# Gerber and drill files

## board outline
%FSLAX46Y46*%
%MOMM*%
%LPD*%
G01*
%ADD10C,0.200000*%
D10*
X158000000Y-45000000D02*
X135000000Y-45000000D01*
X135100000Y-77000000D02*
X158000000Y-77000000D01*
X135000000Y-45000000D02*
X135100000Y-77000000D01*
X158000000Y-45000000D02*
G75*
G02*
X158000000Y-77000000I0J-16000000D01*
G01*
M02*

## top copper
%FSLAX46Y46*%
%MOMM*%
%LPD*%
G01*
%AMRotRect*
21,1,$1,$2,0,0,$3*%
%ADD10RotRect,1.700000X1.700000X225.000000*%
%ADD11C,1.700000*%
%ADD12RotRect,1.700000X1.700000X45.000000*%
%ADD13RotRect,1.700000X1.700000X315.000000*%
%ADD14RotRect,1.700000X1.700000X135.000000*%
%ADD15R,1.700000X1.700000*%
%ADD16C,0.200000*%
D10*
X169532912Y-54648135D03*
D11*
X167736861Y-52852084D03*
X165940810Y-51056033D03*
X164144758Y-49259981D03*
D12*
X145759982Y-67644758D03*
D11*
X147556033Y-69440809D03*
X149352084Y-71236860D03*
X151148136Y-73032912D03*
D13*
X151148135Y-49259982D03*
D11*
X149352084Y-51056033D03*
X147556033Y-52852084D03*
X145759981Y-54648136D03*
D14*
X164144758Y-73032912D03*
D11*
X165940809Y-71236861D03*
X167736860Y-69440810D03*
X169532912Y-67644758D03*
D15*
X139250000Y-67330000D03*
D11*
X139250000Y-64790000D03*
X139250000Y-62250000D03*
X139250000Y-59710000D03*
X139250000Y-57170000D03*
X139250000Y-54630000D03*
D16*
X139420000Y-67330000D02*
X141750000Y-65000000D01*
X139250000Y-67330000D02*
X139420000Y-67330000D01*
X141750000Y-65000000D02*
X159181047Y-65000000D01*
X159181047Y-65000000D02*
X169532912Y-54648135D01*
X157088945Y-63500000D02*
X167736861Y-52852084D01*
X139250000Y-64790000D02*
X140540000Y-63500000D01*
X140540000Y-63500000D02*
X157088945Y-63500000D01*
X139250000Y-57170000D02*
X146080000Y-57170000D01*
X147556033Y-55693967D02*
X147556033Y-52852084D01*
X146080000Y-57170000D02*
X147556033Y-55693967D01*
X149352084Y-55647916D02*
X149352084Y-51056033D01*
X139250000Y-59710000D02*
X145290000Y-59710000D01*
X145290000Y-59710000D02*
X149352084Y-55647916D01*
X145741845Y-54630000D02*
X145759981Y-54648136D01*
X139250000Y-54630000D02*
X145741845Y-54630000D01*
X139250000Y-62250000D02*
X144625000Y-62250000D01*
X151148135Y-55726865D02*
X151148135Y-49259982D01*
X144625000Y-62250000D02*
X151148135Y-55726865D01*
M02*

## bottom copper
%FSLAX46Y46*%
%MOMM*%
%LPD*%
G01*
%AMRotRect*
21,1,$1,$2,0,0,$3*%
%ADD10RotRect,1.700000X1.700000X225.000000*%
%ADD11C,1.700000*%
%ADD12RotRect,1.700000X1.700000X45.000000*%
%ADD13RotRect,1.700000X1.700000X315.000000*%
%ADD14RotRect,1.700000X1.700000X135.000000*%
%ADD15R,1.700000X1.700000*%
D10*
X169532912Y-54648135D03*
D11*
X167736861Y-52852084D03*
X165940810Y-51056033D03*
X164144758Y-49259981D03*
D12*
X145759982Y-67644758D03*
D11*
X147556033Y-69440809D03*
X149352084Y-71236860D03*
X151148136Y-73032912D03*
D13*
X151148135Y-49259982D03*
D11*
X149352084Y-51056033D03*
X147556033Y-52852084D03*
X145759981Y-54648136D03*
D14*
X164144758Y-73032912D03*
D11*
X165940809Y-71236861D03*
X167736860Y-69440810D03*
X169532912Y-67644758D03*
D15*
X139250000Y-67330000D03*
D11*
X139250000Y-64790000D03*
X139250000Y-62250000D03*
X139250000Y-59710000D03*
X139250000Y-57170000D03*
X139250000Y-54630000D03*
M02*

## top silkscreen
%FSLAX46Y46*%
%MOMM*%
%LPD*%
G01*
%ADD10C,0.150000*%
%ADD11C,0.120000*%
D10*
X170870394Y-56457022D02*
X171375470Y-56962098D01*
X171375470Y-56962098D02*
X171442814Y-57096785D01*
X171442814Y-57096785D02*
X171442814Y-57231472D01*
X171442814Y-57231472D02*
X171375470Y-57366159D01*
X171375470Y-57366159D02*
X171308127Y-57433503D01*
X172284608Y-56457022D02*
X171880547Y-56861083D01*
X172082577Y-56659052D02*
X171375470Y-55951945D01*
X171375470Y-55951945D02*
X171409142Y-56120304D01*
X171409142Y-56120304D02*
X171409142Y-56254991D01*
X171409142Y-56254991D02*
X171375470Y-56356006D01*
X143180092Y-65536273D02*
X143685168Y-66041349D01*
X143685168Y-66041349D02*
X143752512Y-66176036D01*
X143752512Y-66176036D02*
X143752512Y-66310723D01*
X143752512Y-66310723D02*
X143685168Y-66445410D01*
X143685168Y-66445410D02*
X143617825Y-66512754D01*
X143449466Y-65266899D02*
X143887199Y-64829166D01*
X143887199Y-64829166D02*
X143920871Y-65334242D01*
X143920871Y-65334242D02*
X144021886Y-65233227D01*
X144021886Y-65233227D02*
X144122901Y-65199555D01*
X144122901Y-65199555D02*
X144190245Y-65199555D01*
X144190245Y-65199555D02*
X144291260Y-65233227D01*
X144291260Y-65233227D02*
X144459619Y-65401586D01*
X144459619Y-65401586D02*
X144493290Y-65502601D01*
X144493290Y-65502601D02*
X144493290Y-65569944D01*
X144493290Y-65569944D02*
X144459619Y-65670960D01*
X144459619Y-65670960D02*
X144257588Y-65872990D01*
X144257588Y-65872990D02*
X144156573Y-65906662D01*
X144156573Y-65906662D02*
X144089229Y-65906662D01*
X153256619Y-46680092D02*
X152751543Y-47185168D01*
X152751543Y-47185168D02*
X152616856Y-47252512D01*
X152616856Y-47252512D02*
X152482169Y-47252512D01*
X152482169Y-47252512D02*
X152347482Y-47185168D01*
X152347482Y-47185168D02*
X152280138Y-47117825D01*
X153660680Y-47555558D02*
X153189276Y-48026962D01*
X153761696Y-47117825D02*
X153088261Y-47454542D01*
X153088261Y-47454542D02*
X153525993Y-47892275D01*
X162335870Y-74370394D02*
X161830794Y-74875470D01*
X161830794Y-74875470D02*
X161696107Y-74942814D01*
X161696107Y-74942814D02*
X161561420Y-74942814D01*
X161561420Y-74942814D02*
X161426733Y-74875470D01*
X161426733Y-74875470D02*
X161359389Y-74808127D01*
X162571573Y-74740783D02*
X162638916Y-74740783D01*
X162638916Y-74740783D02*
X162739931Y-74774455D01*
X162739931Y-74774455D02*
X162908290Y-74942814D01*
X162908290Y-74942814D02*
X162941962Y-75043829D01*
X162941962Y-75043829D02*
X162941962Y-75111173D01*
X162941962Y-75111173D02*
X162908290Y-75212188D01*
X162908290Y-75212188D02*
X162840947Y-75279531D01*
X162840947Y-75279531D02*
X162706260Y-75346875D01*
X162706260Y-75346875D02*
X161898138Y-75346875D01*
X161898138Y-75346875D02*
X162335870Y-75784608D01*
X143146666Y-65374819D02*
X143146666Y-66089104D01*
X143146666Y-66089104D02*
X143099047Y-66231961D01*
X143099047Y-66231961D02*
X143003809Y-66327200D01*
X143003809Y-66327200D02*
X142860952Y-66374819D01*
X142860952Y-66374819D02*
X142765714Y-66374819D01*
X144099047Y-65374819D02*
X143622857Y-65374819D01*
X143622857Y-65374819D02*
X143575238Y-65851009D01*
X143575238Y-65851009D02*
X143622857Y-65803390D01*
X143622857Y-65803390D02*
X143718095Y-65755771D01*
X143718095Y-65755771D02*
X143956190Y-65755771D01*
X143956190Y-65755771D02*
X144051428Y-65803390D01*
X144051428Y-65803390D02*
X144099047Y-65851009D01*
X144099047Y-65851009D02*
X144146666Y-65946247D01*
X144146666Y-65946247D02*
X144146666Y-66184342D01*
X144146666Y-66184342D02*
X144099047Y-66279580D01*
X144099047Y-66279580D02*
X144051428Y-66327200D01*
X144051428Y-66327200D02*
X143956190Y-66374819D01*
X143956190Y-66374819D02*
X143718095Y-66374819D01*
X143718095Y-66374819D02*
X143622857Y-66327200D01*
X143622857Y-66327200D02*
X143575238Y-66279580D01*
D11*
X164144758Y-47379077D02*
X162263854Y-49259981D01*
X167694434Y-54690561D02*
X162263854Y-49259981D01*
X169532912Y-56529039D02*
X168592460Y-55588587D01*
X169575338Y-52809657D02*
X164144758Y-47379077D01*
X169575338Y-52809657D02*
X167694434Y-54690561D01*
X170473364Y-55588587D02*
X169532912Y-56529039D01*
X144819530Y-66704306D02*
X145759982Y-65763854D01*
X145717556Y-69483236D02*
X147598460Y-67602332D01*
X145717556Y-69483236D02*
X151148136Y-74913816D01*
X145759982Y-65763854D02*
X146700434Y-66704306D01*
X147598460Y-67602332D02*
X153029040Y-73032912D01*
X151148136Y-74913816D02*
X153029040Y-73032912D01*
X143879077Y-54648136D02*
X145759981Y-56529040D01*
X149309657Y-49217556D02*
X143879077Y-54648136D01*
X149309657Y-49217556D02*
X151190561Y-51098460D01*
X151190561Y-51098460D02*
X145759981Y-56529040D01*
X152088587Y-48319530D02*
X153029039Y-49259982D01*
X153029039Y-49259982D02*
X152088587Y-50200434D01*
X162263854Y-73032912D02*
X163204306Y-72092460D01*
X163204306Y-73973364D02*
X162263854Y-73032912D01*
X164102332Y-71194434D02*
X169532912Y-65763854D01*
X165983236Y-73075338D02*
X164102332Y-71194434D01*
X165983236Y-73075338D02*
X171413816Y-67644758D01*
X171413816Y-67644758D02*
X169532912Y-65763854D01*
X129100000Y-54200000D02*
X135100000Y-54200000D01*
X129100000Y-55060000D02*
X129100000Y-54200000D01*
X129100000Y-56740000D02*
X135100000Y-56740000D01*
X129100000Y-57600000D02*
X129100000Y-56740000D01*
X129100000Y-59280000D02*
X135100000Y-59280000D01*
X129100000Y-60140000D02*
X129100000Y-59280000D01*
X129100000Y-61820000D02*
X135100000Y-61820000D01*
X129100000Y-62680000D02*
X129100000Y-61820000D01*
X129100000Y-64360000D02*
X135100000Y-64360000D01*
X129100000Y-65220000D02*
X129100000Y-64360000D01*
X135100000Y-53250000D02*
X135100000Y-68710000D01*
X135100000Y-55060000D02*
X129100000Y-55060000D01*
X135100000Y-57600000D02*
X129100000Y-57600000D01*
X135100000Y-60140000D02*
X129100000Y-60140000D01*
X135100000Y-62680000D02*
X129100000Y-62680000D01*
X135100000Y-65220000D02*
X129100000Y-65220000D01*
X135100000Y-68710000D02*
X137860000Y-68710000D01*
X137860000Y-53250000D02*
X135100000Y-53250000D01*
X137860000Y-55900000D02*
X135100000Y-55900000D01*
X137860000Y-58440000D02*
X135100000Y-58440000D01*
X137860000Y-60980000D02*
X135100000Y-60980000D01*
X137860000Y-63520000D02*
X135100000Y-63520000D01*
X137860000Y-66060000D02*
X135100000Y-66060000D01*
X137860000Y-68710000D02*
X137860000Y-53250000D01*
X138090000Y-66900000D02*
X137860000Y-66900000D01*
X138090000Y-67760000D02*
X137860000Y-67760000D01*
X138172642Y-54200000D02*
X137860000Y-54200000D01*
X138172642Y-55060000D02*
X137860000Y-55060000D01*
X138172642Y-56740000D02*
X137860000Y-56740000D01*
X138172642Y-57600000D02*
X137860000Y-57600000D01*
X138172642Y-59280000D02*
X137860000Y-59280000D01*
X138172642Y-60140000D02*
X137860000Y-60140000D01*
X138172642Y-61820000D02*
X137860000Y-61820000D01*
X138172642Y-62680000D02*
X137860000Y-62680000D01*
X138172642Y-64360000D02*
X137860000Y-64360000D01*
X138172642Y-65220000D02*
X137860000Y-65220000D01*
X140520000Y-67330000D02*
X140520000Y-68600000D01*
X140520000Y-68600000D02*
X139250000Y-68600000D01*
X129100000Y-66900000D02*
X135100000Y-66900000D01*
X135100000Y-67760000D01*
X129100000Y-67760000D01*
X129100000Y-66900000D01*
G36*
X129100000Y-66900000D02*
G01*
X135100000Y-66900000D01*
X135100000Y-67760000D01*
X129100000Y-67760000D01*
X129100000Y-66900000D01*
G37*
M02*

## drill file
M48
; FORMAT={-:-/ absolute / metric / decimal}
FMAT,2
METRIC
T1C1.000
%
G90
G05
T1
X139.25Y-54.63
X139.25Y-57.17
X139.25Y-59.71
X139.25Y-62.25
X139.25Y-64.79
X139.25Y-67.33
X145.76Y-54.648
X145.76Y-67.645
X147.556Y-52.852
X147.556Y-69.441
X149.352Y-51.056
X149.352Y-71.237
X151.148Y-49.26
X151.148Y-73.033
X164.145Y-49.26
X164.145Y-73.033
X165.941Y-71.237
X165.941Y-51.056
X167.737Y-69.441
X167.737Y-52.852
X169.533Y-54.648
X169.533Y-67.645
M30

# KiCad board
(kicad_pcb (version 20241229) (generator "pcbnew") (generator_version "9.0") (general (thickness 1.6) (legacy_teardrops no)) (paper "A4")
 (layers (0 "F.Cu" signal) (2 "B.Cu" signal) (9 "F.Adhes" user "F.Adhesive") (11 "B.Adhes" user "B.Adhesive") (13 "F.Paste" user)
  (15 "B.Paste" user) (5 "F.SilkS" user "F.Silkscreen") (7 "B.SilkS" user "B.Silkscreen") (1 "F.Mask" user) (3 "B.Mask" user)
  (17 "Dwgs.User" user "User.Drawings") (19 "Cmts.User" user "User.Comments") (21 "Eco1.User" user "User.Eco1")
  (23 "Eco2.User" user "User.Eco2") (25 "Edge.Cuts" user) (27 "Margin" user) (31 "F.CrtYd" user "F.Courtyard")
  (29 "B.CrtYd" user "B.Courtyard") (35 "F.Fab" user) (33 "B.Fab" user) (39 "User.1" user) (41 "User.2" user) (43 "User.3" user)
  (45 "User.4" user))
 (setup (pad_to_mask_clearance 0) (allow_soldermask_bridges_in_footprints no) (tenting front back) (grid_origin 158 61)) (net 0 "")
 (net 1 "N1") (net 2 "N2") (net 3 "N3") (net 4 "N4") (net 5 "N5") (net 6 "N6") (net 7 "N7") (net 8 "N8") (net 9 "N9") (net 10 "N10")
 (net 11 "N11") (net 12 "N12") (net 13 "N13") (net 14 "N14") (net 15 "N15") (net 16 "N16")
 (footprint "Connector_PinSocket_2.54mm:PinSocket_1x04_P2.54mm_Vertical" (layer "F.Cu") (at 169.532912 54.648135 -135)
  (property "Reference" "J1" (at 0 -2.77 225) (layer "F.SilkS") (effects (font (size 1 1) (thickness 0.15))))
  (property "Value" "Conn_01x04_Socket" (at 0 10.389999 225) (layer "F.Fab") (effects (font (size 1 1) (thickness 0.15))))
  (fp_line (start -1.33 8.95) (end 1.33 8.95) (stroke (width 0.12) (type solid)) (layer "F.SilkS"))
  (fp_line (start 1.33 1.270001) (end 1.33 8.95) (stroke (width 0.12) (type solid)) (layer "F.SilkS"))
  (fp_line (start 1.33 -1.33) (end 1.33 0) (stroke (width 0.12) (type solid)) (layer "F.SilkS"))
  (fp_line (start -1.33 1.270001) (end -1.33 8.95) (stroke (width 0.12) (type solid)) (layer "F.SilkS"))
  (fp_line (start -1.33 1.270001) (end 1.33 1.270001) (stroke (width 0.12) (type solid)) (layer "F.SilkS"))
  (fp_line (start 0 -1.33) (end 1.33 -1.33) (stroke (width 0.12) (type solid)) (layer "F.SilkS"))
  (pad "1" thru_hole rect (at 0 0 225) (size 1.7 1.7) (drill 1) (layers "*.Cu" "*.Mask") (remove_unused_layers no) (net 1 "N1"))
  (pad "2" thru_hole circle (at 0 2.54 225) (size 1.7 1.7) (drill 1) (layers "*.Cu" "*.Mask") (remove_unused_layers no) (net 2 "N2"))
  (pad "3" thru_hole circle (at 0 5.079999 225) (size 1.7 1.7) (drill 1) (layers "*.Cu" "*.Mask") (remove_unused_layers no) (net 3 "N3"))
  (pad "4" thru_hole circle (at 0 7.62 225) (size 1.7 1.7) (drill 1) (layers "*.Cu" "*.Mask") (remove_unused_layers no) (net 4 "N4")))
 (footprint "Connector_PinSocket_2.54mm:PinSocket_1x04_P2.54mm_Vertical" (layer "F.Cu") (at 145.759982 67.644758 45)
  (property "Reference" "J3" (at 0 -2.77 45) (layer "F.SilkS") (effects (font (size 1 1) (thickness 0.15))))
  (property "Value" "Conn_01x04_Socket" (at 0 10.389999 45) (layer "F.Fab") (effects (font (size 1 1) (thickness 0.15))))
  (fp_line (start 0 -1.33) (end 1.33 -1.33) (stroke (width 0.12) (type solid)) (layer "F.SilkS"))
  (fp_line (start -1.33 1.270001) (end 1.33 1.270001) (stroke (width 0.12) (type solid)) (layer "F.SilkS"))
  (fp_line (start -1.33 1.270001) (end -1.33 8.95) (stroke (width 0.12) (type solid)) (layer "F.SilkS"))
  (fp_line (start 1.33 -1.33) (end 1.33 0) (stroke (width 0.12) (type solid)) (layer "F.SilkS"))
  (fp_line (start 1.33 1.270001) (end 1.33 8.95) (stroke (width 0.12) (type solid)) (layer "F.SilkS"))
  (fp_line (start -1.33 8.95) (end 1.33 8.95) (stroke (width 0.12) (type solid)) (layer "F.SilkS"))
  (pad "1" thru_hole rect (at 0 0 45) (size 1.7 1.7) (drill 1) (layers "*.Cu" "*.Mask") (remove_unused_layers no) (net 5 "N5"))
  (pad "2" thru_hole circle (at 0 2.54 45) (size 1.7 1.7) (drill 1) (layers "*.Cu" "*.Mask") (remove_unused_layers no) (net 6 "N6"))
  (pad "3" thru_hole circle (at 0 5.079999 45) (size 1.7 1.7) (drill 1) (layers "*.Cu" "*.Mask") (remove_unused_layers no) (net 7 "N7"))
  (pad "4" thru_hole circle (at 0 7.62 45) (size 1.7 1.7) (drill 1) (layers "*.Cu" "*.Mask") (remove_unused_layers no) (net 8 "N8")))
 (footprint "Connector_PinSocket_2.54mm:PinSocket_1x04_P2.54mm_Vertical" (layer "F.Cu") (at 151.148135 49.259982 -45)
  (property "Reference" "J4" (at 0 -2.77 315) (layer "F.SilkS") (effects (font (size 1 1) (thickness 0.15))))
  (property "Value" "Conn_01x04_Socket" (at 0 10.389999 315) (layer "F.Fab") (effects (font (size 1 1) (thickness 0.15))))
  (fp_line (start -1.33 8.95) (end 1.33 8.95) (stroke (width 0.12) (type solid)) (layer "F.SilkS"))
  (fp_line (start -1.33 1.270001) (end -1.33 8.95) (stroke (width 0.12) (type solid)) (layer "F.SilkS"))
  (fp_line (start -1.33 1.270001) (end 1.33 1.270001) (stroke (width 0.12) (type solid)) (layer "F.SilkS"))
  (fp_line (start 1.33 1.270001) (end 1.33 8.95) (stroke (width 0.12) (type solid)) (layer "F.SilkS"))
  (fp_line (start 0 -1.33) (end 1.33 -1.33) (stroke (width 0.12) (type solid)) (layer "F.SilkS"))
  (fp_line (start 1.33 -1.33) (end 1.33 0) (stroke (width 0.12) (type solid)) (layer "F.SilkS"))
  (pad "1" thru_hole rect (at 0 0 315) (size 1.7 1.7) (drill 1) (layers "*.Cu" "*.Mask") (remove_unused_layers no) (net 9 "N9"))
  (pad "2" thru_hole circle (at 0 2.54 315) (size 1.7 1.7) (drill 1) (layers "*.Cu" "*.Mask") (remove_unused_layers no) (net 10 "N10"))
  (pad "3" thru_hole circle (at 0 5.079999 315) (size 1.7 1.7) (drill 1) (layers "*.Cu" "*.Mask") (remove_unused_layers no) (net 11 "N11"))
  (pad "4" thru_hole circle (at 0 7.62 315) (size 1.7 1.7) (drill 1) (layers "*.Cu" "*.Mask") (remove_unused_layers no) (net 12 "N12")))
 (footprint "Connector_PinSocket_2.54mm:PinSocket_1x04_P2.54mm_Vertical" (layer "F.Cu") (at 164.144758 73.032912 135)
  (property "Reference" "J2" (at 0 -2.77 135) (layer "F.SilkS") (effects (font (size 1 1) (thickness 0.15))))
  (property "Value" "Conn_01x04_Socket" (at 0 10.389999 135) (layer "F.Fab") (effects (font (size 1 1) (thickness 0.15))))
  (fp_line (start 1.33 -1.33) (end 1.33 0) (stroke (width 0.12) (type solid)) (layer "F.SilkS"))
  (fp_line (start 0 -1.33) (end 1.33 -1.33) (stroke (width 0.12) (type solid)) (layer "F.SilkS"))
  (fp_line (start 1.33 1.270001) (end 1.33 8.95) (stroke (width 0.12) (type solid)) (layer "F.SilkS"))
  (fp_line (start -1.33 1.270001) (end 1.33 1.270001) (stroke (width 0.12) (type solid)) (layer "F.SilkS"))
  (fp_line (start -1.33 1.270001) (end -1.33 8.95) (stroke (width 0.12) (type solid)) (layer "F.SilkS"))
  (fp_line (start -1.33 8.95) (end 1.33 8.95) (stroke (width 0.12) (type solid)) (layer "F.SilkS"))
  (pad "1" thru_hole rect (at 0 0 135) (size 1.7 1.7) (drill 1) (layers "*.Cu" "*.Mask") (remove_unused_layers no) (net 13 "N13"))
  (pad "2" thru_hole circle (at 0 2.54 135) (size 1.7 1.7) (drill 1) (layers "*.Cu" "*.Mask") (remove_unused_layers no) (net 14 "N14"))
  (pad "3" thru_hole circle (at 0 5.079999 135) (size 1.7 1.7) (drill 1) (layers "*.Cu" "*.Mask") (remove_unused_layers no) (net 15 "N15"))
  (pad "4" thru_hole circle (at 0 7.62 135) (size 1.7 1.7) (drill 1) (layers "*.Cu" "*.Mask") (remove_unused_layers no) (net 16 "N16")))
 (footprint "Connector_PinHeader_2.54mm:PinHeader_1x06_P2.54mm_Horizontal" (layer "F.Cu") (at 139.25 67.33 180)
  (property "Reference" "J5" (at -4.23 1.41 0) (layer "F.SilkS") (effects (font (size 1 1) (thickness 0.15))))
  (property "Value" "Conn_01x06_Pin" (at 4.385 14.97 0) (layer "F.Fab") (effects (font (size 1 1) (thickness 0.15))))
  (fp_line (start 10.15 13.13) (end 4.15 13.13) (stroke (width 0.12) (type solid)) (layer "F.SilkS"))
  (fp_line (start 10.15 12.27) (end 10.15 13.13) (stroke (width 0.12) (type solid)) (layer "F.SilkS"))
  (fp_line (start 10.15 10.59) (end 4.15 10.59) (stroke (width 0.12) (type solid)) (layer "F.SilkS"))
  (fp_line (start 10.15 9.73) (end 10.15 10.59) (stroke (width 0.12) (type solid)) (layer "F.SilkS"))
  (fp_line (start 10.15 8.05) (end 4.15 8.05) (stroke (width 0.12) (type solid)) (layer "F.SilkS"))
  (fp_line (start 10.15 7.19) (end 10.15 8.05) (stroke (width 0.12) (type solid)) (layer "F.SilkS"))
  (fp_line (start 10.15 5.51) (end 4.15 5.51) (stroke (width 0.12) (type solid)) (layer "F.SilkS"))
  (fp_line (start 10.15 4.65) (end 10.15 5.51) (stroke (width 0.12) (type solid)) (layer "F.SilkS"))
  (fp_line (start 10.15 2.97) (end 4.15 2.97) (stroke (width 0.12) (type solid)) (layer "F.SilkS"))
  (fp_line (start 10.15 2.11) (end 10.15 2.97) (stroke (width 0.12) (type solid)) (layer "F.SilkS"))
  (fp_line (start 4.15 14.08) (end 4.15 -1.38) (stroke (width 0.12) (type solid)) (layer "F.SilkS"))
  (fp_line (start 4.15 12.27) (end 10.15 12.27) (stroke (width 0.12) (type solid)) (layer "F.SilkS"))
  (fp_line (start 4.15 9.73) (end 10.15 9.73) (stroke (width 0.12) (type solid)) (layer "F.SilkS"))
  (fp_line (start 4.15 7.19) (end 10.15 7.19) (stroke (width 0.12) (type solid)) (layer "F.SilkS"))
  (fp_line (start 4.15 4.65) (end 10.15 4.65) (stroke (width 0.12) (type solid)) (layer "F.SilkS"))
  (fp_line (start 4.15 2.11) (end 10.15 2.11) (stroke (width 0.12) (type solid)) (layer "F.SilkS"))
  (fp_line (start 4.15 -1.38) (end 1.39 -1.38) (stroke (width 0.12) (type solid)) (layer "F.SilkS"))
  (fp_line (start 1.39 14.08) (end 4.15 14.08) (stroke (width 0.12) (type solid)) (layer "F.SilkS"))
  (fp_line (start 1.39 11.43) (end 4.15 11.43) (stroke (width 0.12) (type solid)) (layer "F.SilkS"))
  (fp_line (start 1.39 8.89) (end 4.15 8.89) (stroke (width 0.12) (type solid)) (layer "F.SilkS"))
  (fp_line (start 1.39 6.35) (end 4.15 6.35) (stroke (width 0.12) (type solid)) (layer "F.SilkS"))
  (fp_line (start 1.39 3.81) (end 4.15 3.81) (stroke (width 0.12) (type solid)) (layer "F.SilkS"))
  (fp_line (start 1.39 1.27) (end 4.15 1.27) (stroke (width 0.12) (type solid)) (layer "F.SilkS"))
  (fp_line (start 1.39 -1.38) (end 1.39 14.08) (stroke (width 0.12) (type solid)) (layer "F.SilkS"))
  (fp_line (start 1.16 0.43) (end 1.39 0.43) (stroke (width 0.12) (type solid)) (layer "F.SilkS"))
  (fp_line (start 1.16 -0.43) (end 1.39 -0.43) (stroke (width 0.12) (type solid)) (layer "F.SilkS"))
  (fp_line (start 1.077358 13.13) (end 1.39 13.13) (stroke (width 0.12) (type solid)) (layer "F.SilkS"))
  (fp_line (start 1.077358 12.27) (end 1.39 12.27) (stroke (width 0.12) (type solid)) (layer "F.SilkS"))
  (fp_line (start 1.077358 10.59) (end 1.39 10.59) (stroke (width 0.12) (type solid)) (layer "F.SilkS"))
  (fp_line (start 1.077358 9.73) (end 1.39 9.73) (stroke (width 0.12) (type solid)) (layer "F.SilkS"))
  (fp_line (start 1.077358 8.05) (end 1.39 8.05) (stroke (width 0.12) (type solid)) (layer "F.SilkS"))
  (fp_line (start 1.077358 7.19) (end 1.39 7.19) (stroke (width 0.12) (type solid)) (layer "F.SilkS"))
  (fp_line (start 1.077358 5.51) (end 1.39 5.51) (stroke (width 0.12) (type solid)) (layer "F.SilkS"))
  (fp_line (start 1.077358 4.65) (end 1.39 4.65) (stroke (width 0.12) (type solid)) (layer "F.SilkS"))
  (fp_line (start 1.077358 2.97) (end 1.39 2.97) (stroke (width 0.12) (type solid)) (layer "F.SilkS"))
  (fp_line (start 1.077358 2.11) (end 1.39 2.11) (stroke (width 0.12) (type solid)) (layer "F.SilkS"))
  (fp_line (start -1.27 0) (end -1.27 -1.27) (stroke (width 0.12) (type solid)) (layer "F.SilkS"))
  (fp_line (start -1.27 -1.27) (end 0 -1.27) (stroke (width 0.12) (type solid)) (layer "F.SilkS"))
  (fp_rect (start 4.15 -0.43) (end 10.15 0.43) (stroke (width 0.12) (type solid)) (fill yes) (layer "F.SilkS"))
  (pad "1" thru_hole rect (at 0 0 180) (size 1.7 1.7) (drill 1) (layers "*.Cu" "*.Mask") (remove_unused_layers no) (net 1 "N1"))
  (pad "2" thru_hole circle (at 0 2.54 180) (size 1.7 1.7) (drill 1) (layers "*.Cu" "*.Mask") (remove_unused_layers no) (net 2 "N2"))
  (pad "3" thru_hole circle (at 0 5.08 180) (size 1.7 1.7) (drill 1) (layers "*.Cu" "*.Mask") (remove_unused_layers no) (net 9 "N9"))
  (pad "4" thru_hole circle (at 0 7.62 180) (size 1.7 1.7) (drill 1) (layers "*.Cu" "*.Mask") (remove_unused_layers no) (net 10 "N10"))
  (pad "5" thru_hole circle (at 0 10.16 180) (size 1.7 1.7) (drill 1) (layers "*.Cu" "*.Mask") (remove_unused_layers no) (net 11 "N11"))
  (pad "6" thru_hole circle (at 0 12.7 180) (size 1.7 1.7) (drill 1) (layers "*.Cu" "*.Mask") (remove_unused_layers no) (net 12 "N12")))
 (gr_line (start 158 45) (end 135 45) (stroke (width 0.2) (type solid)) (layer "Edge.Cuts"))
 (gr_line (start 135.1 77) (end 158 77) (stroke (width 0.2) (type solid)) (layer "Edge.Cuts"))
 (gr_line (start 135 45) (end 135.1 77) (stroke (width 0.2) (type solid)) (layer "Edge.Cuts"))
 (gr_arc (start 158 45) (mid 174 61) (end 158 77) (stroke (width 0.2) (type solid)) (layer "Edge.Cuts"))
 (segment (start 139.42 67.33) (end 141.75 65) (width 0.2) (layer "F.Cu") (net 1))
 (segment (start 139.25 67.33) (end 139.42 67.33) (width 0.2) (layer "F.Cu") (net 1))
 (segment (start 141.75 65) (end 159.181047 65) (width 0.2) (layer "F.Cu") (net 1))
 (segment (start 159.181047 65) (end 169.532912 54.648135) (width 0.2) (layer "F.Cu") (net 1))
 (segment (start 157.088945 63.5) (end 167.736861 52.852084) (width 0.2) (layer "F.Cu") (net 2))
 (segment (start 139.25 64.79) (end 140.54 63.5) (width 0.2) (layer "F.Cu") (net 2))
 (segment (start 140.54 63.5) (end 157.088945 63.5) (width 0.2) (layer "F.Cu") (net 2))
 (segment (start 139.25 57.17) (end 146.08 57.17) (width 0.2) (layer "F.Cu") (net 11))
 (segment (start 147.556033 55.693967) (end 147.556033 52.852084) (width 0.2) (layer "F.Cu") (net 11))
 (segment (start 146.08 57.17) (end 147.556033 55.693967) (width 0.2) (layer "F.Cu") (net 11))
 (segment (start 149.352084 55.647916) (end 149.352084 51.056033) (width 0.2) (layer "F.Cu") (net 10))
 (segment (start 139.25 59.71) (end 145.29 59.71) (width 0.2) (layer "F.Cu") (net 10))
 (segment (start 145.29 59.71) (end 149.352084 55.647916) (width 0.2) (layer "F.Cu") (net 10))
 (segment (start 145.741845 54.63) (end 145.759981 54.648136) (width 0.2) (layer "F.Cu") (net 12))
 (segment (start 139.25 54.63) (end 145.741845 54.63) (width 0.2) (layer "F.Cu") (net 12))
 (segment (start 139.25 62.25) (end 144.625 62.25) (width 0.2) (layer "F.Cu") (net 9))
 (segment (start 151.148135 55.726865) (end 151.148135 49.259982) (width 0.2) (layer "F.Cu") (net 9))
 (segment (start 144.625 62.25) (end 151.148135 55.726865) (width 0.2) (layer "F.Cu") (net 9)))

